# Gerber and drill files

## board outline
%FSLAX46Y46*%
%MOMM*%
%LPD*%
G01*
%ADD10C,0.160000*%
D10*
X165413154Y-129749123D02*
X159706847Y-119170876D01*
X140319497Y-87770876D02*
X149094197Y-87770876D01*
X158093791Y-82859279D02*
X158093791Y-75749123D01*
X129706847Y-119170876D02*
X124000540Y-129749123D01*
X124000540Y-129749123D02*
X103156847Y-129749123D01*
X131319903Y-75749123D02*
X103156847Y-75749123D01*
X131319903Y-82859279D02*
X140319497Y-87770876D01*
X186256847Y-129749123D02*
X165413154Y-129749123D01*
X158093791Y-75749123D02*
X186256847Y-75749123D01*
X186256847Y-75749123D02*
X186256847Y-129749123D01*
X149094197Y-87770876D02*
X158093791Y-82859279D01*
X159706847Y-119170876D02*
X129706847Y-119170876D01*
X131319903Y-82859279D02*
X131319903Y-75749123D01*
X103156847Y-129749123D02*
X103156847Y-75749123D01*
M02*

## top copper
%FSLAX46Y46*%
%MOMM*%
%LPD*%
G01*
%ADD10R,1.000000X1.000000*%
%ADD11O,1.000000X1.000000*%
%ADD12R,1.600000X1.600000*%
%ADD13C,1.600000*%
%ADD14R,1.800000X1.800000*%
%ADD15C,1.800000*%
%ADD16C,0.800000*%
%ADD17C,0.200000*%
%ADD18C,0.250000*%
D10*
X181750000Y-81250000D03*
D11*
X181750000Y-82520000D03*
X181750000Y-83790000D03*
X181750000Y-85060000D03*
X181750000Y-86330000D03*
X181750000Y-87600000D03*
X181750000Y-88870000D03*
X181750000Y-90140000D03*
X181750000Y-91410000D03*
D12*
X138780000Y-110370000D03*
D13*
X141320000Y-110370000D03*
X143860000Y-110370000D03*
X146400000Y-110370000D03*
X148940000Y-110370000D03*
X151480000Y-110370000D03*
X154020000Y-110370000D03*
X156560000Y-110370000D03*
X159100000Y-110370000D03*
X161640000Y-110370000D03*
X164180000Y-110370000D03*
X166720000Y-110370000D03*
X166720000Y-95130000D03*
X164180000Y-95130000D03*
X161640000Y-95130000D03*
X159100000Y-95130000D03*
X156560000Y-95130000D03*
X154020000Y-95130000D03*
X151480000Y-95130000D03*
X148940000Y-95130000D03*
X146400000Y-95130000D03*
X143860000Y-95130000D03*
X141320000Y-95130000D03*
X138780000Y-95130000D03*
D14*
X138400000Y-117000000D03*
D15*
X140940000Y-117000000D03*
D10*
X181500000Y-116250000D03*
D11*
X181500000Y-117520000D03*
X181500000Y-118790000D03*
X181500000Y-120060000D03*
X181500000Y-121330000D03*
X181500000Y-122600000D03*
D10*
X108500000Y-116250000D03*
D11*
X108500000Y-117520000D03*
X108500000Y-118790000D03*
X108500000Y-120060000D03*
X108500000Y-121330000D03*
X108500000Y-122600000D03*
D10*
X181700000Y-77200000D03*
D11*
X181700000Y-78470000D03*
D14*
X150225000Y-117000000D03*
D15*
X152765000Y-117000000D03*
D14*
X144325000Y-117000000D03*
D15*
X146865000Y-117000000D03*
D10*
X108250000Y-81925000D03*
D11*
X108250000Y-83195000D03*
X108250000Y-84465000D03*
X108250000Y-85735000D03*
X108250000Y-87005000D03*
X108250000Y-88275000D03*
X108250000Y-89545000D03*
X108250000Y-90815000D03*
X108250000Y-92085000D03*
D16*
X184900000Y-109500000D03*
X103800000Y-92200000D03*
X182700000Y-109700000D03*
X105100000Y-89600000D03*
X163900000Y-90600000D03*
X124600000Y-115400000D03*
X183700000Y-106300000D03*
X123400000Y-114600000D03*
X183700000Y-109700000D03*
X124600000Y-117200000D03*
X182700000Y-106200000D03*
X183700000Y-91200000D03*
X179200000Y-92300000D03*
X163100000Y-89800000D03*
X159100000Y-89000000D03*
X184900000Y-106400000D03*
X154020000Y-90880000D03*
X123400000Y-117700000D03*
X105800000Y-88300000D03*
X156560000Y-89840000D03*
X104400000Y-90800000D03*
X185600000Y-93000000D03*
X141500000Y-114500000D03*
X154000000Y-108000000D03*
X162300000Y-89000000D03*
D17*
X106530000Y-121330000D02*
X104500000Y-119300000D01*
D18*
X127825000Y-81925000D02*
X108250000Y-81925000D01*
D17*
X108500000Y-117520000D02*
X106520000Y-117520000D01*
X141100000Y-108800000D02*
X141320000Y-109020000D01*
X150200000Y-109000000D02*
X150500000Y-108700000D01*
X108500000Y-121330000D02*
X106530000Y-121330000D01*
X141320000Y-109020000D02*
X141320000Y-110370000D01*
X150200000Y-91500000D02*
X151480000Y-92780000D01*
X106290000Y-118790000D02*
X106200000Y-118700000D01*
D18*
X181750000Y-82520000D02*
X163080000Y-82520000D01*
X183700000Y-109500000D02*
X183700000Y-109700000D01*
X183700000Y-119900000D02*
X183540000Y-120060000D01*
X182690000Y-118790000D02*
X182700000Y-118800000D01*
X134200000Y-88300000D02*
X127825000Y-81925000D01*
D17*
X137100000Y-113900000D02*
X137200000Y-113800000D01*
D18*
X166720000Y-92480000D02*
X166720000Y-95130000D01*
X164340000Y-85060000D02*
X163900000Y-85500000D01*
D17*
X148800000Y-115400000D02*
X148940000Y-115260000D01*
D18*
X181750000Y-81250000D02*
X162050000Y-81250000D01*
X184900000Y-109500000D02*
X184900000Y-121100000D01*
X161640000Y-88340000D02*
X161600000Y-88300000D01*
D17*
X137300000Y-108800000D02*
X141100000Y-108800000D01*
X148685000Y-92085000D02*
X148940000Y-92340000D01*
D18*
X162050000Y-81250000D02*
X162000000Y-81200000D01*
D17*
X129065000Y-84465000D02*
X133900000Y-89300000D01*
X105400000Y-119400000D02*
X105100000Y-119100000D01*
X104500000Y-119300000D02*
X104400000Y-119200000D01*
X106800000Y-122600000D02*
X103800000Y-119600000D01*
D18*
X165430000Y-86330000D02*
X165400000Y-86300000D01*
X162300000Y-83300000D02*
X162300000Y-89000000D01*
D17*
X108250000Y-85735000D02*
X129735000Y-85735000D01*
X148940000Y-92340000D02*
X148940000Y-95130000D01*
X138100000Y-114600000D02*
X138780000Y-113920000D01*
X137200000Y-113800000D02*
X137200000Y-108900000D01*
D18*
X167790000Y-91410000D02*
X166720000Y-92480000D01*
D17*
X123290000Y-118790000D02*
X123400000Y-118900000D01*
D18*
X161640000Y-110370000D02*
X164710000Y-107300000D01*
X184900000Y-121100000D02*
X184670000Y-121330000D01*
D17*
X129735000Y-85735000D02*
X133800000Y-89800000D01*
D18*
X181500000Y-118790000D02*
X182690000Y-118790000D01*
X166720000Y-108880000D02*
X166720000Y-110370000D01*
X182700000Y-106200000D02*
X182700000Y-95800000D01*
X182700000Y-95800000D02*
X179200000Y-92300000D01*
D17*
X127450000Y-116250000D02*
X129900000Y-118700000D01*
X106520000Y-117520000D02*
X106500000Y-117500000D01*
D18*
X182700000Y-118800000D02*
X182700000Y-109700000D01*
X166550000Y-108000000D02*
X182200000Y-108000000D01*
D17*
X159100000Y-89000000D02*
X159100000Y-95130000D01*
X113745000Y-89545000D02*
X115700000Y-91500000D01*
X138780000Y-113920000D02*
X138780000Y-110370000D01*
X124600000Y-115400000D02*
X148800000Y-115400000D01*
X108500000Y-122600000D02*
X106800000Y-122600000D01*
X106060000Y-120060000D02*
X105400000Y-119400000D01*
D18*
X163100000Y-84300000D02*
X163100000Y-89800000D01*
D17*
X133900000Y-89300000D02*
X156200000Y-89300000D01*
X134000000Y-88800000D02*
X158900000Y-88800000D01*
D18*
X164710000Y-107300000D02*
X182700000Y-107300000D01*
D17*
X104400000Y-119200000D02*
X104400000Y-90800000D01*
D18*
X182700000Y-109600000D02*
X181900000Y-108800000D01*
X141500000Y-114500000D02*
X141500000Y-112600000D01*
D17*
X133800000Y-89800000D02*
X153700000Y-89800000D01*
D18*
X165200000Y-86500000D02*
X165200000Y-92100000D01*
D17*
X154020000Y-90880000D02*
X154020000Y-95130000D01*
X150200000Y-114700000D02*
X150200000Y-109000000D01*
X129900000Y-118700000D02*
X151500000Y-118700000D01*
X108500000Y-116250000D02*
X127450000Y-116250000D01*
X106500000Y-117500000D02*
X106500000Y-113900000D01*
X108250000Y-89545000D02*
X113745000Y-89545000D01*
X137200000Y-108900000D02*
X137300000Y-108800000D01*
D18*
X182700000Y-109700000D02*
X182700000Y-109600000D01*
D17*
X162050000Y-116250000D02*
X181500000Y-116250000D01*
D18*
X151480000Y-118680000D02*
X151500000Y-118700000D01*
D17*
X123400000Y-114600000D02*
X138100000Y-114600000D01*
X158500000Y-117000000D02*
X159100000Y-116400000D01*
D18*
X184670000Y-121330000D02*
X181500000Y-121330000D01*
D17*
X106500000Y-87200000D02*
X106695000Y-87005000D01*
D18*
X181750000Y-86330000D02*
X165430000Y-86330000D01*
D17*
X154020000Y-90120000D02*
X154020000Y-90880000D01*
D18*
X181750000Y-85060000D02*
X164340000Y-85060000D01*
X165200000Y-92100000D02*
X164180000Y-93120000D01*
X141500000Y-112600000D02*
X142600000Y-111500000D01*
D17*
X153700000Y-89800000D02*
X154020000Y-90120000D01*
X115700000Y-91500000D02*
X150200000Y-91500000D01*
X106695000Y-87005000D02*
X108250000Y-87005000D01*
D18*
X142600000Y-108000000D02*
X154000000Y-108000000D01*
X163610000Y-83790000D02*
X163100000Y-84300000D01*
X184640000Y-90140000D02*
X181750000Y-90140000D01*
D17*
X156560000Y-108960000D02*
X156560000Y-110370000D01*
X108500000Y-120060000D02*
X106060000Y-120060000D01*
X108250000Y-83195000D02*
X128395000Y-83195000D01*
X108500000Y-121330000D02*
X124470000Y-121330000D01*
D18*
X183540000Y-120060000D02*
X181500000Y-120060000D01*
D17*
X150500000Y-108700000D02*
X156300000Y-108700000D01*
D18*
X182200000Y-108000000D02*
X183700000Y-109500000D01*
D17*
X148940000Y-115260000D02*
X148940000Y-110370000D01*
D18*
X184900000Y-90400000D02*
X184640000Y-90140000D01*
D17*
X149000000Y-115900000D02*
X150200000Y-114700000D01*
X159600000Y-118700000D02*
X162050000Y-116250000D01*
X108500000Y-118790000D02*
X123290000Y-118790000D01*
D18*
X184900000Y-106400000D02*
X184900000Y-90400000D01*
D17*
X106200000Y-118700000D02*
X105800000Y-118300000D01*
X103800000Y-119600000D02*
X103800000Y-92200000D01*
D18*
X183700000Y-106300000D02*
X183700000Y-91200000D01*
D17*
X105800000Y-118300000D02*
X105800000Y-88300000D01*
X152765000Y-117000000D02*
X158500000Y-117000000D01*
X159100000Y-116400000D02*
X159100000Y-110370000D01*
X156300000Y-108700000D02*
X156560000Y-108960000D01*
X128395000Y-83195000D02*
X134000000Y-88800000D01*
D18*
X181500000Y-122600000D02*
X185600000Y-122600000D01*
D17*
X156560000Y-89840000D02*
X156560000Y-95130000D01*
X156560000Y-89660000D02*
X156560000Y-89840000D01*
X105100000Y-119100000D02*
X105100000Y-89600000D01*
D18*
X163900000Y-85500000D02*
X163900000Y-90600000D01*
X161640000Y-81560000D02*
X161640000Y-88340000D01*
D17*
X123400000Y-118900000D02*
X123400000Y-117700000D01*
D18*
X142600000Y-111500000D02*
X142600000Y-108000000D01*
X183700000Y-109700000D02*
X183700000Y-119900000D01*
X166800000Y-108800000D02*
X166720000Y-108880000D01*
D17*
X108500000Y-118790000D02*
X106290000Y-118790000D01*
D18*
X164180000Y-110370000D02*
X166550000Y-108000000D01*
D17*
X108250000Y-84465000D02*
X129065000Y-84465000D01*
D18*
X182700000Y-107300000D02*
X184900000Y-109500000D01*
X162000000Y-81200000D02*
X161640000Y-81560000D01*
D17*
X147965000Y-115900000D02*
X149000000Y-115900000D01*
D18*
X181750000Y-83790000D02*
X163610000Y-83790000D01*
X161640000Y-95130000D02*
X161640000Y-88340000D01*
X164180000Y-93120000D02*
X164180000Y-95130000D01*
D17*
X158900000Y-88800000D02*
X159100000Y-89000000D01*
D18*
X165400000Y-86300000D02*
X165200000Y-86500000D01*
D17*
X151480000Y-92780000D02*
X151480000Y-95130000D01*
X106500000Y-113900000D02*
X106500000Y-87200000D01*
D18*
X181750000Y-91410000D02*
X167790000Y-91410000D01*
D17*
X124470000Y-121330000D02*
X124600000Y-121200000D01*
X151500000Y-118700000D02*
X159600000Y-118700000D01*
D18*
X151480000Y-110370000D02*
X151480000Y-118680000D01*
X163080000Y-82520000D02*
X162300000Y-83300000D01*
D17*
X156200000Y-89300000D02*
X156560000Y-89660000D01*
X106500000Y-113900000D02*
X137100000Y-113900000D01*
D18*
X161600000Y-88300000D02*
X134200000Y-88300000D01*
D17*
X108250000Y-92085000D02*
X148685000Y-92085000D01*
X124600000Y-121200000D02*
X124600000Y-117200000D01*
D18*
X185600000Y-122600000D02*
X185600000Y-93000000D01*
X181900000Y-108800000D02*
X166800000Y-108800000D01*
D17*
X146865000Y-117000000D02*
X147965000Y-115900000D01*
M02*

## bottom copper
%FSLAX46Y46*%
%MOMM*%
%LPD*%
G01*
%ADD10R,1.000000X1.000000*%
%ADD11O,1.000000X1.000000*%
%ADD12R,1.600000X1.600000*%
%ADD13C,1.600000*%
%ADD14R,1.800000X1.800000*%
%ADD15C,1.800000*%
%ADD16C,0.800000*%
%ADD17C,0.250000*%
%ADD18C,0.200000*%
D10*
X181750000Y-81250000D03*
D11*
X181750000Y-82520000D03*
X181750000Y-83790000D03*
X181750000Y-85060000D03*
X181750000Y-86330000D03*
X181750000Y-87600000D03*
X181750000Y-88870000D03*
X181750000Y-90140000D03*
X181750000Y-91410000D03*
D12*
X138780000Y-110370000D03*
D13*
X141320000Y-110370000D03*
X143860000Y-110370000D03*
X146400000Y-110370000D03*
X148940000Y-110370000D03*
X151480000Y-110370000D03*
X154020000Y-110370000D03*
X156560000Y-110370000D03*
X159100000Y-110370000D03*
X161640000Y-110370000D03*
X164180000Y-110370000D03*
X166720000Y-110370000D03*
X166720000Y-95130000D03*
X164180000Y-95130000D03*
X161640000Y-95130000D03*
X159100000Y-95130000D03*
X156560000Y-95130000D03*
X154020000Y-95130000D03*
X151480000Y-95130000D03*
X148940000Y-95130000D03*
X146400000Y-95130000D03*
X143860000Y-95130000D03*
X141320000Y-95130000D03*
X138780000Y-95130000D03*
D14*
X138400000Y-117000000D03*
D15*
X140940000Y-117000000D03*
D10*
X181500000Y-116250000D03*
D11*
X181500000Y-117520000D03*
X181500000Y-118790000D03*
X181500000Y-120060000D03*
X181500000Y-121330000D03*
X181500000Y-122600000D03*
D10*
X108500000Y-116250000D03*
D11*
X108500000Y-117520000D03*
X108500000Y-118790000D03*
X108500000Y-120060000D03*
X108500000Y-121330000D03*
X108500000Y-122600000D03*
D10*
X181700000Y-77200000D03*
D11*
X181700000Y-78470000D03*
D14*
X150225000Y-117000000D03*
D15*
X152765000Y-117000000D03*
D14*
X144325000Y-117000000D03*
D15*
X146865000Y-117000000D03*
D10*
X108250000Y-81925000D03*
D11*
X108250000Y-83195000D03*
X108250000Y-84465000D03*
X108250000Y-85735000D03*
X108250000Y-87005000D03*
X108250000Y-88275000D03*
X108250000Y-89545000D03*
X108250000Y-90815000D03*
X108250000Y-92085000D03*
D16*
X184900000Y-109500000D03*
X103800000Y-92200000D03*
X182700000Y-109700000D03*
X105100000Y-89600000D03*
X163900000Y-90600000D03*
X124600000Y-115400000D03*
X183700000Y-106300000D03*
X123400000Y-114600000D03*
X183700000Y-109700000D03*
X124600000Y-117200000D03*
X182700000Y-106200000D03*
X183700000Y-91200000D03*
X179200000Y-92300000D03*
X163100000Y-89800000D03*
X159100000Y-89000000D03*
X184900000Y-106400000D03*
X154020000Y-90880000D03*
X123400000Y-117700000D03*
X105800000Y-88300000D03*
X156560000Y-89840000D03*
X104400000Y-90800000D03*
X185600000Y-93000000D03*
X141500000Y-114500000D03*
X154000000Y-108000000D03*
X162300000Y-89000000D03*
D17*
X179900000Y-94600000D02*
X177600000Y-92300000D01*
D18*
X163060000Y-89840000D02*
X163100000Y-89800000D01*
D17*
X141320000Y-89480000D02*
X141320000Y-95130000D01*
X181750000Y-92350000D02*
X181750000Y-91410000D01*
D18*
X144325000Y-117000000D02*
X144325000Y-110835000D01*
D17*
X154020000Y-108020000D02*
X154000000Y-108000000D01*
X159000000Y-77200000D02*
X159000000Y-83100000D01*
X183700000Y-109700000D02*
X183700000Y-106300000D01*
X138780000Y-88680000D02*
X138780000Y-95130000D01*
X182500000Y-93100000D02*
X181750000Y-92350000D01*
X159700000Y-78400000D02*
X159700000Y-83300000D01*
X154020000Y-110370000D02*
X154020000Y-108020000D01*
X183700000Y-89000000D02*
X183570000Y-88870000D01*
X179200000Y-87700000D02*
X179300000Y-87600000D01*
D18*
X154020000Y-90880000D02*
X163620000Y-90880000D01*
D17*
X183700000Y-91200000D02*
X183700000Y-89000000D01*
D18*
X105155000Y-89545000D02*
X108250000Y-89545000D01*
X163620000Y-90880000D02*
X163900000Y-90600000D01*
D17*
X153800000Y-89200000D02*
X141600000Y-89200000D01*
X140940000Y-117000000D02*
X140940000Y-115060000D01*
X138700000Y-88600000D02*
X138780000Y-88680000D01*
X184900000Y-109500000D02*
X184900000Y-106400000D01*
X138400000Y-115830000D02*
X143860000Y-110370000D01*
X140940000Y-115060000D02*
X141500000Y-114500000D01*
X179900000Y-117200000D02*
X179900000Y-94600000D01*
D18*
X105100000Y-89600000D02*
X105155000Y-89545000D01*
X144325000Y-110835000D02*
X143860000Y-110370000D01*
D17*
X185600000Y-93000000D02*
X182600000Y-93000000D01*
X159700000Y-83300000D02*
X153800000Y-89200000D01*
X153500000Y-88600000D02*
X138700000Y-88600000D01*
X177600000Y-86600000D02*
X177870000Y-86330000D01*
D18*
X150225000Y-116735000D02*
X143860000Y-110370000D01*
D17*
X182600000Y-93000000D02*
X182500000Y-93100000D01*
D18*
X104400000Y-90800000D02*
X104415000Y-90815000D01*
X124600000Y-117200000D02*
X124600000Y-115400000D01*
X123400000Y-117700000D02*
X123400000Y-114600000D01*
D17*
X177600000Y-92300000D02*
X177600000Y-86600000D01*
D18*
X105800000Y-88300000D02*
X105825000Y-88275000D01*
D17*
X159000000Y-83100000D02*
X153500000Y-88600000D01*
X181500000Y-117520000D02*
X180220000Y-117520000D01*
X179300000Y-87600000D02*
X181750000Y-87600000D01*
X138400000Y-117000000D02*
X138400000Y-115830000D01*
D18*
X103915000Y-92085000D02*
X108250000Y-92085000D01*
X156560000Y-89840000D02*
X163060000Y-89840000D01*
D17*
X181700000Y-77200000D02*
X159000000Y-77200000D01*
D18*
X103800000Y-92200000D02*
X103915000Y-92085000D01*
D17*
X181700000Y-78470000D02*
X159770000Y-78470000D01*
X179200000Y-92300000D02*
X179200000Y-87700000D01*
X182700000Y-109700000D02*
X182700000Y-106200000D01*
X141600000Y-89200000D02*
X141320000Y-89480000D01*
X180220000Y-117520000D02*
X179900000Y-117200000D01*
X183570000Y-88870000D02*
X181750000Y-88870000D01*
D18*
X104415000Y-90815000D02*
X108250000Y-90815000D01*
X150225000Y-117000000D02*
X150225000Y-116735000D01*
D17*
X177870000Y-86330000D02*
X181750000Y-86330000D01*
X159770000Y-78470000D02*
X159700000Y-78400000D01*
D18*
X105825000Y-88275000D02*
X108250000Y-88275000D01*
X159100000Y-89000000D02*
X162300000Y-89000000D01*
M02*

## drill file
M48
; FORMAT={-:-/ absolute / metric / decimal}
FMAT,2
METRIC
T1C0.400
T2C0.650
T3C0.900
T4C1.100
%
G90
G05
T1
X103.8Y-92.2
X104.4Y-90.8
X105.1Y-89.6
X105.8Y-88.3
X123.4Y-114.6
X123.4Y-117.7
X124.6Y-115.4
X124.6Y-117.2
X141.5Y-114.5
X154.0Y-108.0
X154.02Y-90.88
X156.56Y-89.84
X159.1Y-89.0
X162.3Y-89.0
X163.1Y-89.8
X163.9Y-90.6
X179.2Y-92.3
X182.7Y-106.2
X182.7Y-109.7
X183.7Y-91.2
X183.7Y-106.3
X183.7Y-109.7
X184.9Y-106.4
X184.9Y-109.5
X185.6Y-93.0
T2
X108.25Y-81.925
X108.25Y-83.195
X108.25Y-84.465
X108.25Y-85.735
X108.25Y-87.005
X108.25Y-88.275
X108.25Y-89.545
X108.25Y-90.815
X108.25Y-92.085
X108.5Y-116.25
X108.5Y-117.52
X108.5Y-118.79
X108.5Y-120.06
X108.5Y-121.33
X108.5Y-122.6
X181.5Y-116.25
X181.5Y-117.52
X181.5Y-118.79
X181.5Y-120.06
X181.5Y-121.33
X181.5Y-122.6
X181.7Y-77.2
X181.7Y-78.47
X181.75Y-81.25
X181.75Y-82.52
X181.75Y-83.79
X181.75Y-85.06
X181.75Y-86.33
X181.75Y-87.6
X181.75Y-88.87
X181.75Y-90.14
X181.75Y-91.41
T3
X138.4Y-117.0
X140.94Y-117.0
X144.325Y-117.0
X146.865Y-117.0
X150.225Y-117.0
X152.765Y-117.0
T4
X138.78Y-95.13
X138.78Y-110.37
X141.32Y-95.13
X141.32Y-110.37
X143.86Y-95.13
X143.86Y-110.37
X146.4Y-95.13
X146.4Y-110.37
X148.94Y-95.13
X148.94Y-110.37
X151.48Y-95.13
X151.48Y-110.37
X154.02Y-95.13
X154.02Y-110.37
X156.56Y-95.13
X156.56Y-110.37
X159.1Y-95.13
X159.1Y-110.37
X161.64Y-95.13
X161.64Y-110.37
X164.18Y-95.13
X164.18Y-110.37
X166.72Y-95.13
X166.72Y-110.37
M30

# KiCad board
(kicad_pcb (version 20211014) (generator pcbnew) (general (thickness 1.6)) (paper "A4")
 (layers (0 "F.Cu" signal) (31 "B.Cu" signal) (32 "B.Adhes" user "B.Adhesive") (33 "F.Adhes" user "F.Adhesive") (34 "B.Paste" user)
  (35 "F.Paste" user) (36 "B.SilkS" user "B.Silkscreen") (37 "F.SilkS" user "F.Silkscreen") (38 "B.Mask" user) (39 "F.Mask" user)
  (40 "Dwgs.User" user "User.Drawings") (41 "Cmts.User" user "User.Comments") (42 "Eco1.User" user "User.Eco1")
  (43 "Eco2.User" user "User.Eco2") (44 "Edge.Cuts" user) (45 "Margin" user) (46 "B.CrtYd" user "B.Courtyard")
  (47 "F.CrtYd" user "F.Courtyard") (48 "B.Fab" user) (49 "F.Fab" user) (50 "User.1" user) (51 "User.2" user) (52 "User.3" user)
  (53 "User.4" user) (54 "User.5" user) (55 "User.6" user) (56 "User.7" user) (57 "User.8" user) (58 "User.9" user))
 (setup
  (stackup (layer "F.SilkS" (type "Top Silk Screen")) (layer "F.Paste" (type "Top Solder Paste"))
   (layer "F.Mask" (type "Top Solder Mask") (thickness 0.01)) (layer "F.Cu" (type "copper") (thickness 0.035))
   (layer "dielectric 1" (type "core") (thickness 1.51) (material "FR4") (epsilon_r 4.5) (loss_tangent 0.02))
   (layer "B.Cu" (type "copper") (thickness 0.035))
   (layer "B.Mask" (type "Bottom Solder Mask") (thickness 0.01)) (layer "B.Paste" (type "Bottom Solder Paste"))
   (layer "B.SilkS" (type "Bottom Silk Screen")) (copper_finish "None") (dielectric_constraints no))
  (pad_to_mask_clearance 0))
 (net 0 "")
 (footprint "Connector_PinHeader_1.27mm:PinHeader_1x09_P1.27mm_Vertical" (layer "F.Cu") (at 181.75 81.25)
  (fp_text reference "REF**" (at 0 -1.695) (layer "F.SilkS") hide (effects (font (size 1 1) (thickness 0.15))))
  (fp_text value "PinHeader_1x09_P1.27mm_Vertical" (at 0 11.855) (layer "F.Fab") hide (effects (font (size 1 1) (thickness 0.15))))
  (pad "1" thru_hole rect (at 0 0) (size 1 1) (drill 0.65) (layers *.Cu *.Mask))
  (pad "2" thru_hole oval (at 0 1.27) (size 1 1) (drill 0.65) (layers *.Cu *.Mask))
  (pad "3" thru_hole oval (at 0 2.54) (size 1 1) (drill 0.65) (layers *.Cu *.Mask))
  (pad "4" thru_hole oval (at 0 3.81) (size 1 1) (drill 0.65) (layers *.Cu *.Mask))
  (pad "5" thru_hole oval (at 0 5.08) (size 1 1) (drill 0.65) (layers *.Cu *.Mask))
  (pad "6" thru_hole oval (at 0 6.35) (size 1 1) (drill 0.65) (layers *.Cu *.Mask))
  (pad "7" thru_hole oval (at 0 7.62) (size 1 1) (drill 0.65) (layers *.Cu *.Mask))
  (pad "8" thru_hole oval (at 0 8.89) (size 1 1) (drill 0.65) (layers *.Cu *.Mask))
  (pad "9" thru_hole oval (at 0 10.16) (size 1 1) (drill 0.65) (layers *.Cu *.Mask)))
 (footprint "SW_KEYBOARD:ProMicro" (layer "F.Cu") (at 152.75 102.75)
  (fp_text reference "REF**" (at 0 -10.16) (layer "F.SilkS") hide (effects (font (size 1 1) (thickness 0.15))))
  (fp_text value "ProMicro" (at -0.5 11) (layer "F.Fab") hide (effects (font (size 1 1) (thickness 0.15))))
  (pad "1" thru_hole rect locked (at -13.97 7.62) (size 1.6 1.6) (drill 1.1) (layers *.Cu *.Mask "F.SilkS"))
  (pad "2" thru_hole circle locked (at -11.43 7.62) (size 1.6 1.6) (drill 1.1) (layers *.Cu *.Mask "F.SilkS"))
  (pad "3" thru_hole circle locked (at -8.89 7.62) (size 1.6 1.6) (drill 1.1) (layers *.Cu *.Mask "F.SilkS"))
  (pad "4" thru_hole circle locked (at -6.35 7.62) (size 1.6 1.6) (drill 1.1) (layers *.Cu *.Mask "F.SilkS"))
  (pad "5" thru_hole circle locked (at -3.81 7.62) (size 1.6 1.6) (drill 1.1) (layers *.Cu *.Mask "F.SilkS"))
  (pad "6" thru_hole circle locked (at -1.27 7.62) (size 1.6 1.6) (drill 1.1) (layers *.Cu *.Mask "F.SilkS"))
  (pad "7" thru_hole circle locked (at 1.27 7.62) (size 1.6 1.6) (drill 1.1) (layers *.Cu *.Mask "F.SilkS"))
  (pad "8" thru_hole circle locked (at 3.81 7.62) (size 1.6 1.6) (drill 1.1) (layers *.Cu *.Mask "F.SilkS"))
  (pad "9" thru_hole circle locked (at 6.35 7.62) (size 1.6 1.6) (drill 1.1) (layers *.Cu *.Mask "F.SilkS"))
  (pad "10" thru_hole circle locked (at 8.89 7.62) (size 1.6 1.6) (drill 1.1) (layers *.Cu *.Mask "F.SilkS"))
  (pad "11" thru_hole circle locked (at 11.43 7.62) (size 1.6 1.6) (drill 1.1) (layers *.Cu *.Mask "F.SilkS"))
  (pad "12" thru_hole circle locked (at 13.97 7.62) (size 1.6 1.6) (drill 1.1) (layers *.Cu *.Mask "F.SilkS"))
  (pad "13" thru_hole circle locked (at 13.97 -7.62) (size 1.6 1.6) (drill 1.1) (layers *.Cu *.Mask "F.SilkS"))
  (pad "14" thru_hole circle locked (at 11.43 -7.62) (size 1.6 1.6) (drill 1.1) (layers *.Cu *.Mask "F.SilkS"))
  (pad "15" thru_hole circle locked (at 8.89 -7.62) (size 1.6 1.6) (drill 1.1) (layers *.Cu *.Mask "F.SilkS"))
  (pad "16" thru_hole circle locked (at 6.35 -7.62) (size 1.6 1.6) (drill 1.1) (layers *.Cu *.Mask "F.SilkS"))
  (pad "17" thru_hole circle locked (at 3.81 -7.62) (size 1.6 1.6) (drill 1.1) (layers *.Cu *.Mask "F.SilkS"))
  (pad "18" thru_hole circle locked (at 1.27 -7.62) (size 1.6 1.6) (drill 1.1) (layers *.Cu *.Mask "F.SilkS"))
  (pad "19" thru_hole circle locked (at -1.27 -7.62) (size 1.6 1.6) (drill 1.1) (layers *.Cu *.Mask "F.SilkS"))
  (pad "20" thru_hole circle locked (at -3.81 -7.62) (size 1.6 1.6) (drill 1.1) (layers *.Cu *.Mask "F.SilkS"))
  (pad "21" thru_hole circle locked (at -6.35 -7.62) (size 1.6 1.6) (drill 1.1) (layers *.Cu *.Mask "F.SilkS"))
  (pad "22" thru_hole circle locked (at -8.89 -7.62) (size 1.6 1.6) (drill 1.1) (layers *.Cu *.Mask "F.SilkS"))
  (pad "23" thru_hole circle locked (at -11.43 -7.62) (size 1.6 1.6) (drill 1.1) (layers *.Cu *.Mask "F.SilkS"))
  (pad "24" thru_hole circle locked (at -13.97 -7.62) (size 1.6 1.6) (drill 1.1) (layers *.Cu *.Mask "F.SilkS")))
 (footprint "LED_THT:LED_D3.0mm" (layer "F.Cu") (at 138.4 117)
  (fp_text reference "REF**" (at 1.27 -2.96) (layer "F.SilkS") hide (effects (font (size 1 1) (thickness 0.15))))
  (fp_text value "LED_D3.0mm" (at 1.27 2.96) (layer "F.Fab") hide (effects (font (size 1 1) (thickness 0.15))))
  (pad "1" thru_hole rect (at 0 0) (size 1.8 1.8) (drill 0.9) (layers *.Cu *.Mask))
  (pad "2" thru_hole circle (at 2.54 0) (size 1.8 1.8) (drill 0.9) (layers *.Cu *.Mask)))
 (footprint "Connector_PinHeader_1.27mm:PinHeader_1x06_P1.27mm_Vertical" (layer "F.Cu") (at 181.5 116.25)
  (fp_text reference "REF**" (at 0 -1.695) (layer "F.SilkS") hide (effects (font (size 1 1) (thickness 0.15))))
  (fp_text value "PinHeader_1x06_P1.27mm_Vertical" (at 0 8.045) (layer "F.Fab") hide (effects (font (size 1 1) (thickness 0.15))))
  (pad "1" thru_hole rect (at 0 0) (size 1 1) (drill 0.65) (layers *.Cu *.Mask))
  (pad "2" thru_hole oval (at 0 1.27) (size 1 1) (drill 0.65) (layers *.Cu *.Mask))
  (pad "3" thru_hole oval (at 0 2.54) (size 1 1) (drill 0.65) (layers *.Cu *.Mask))
  (pad "4" thru_hole oval (at 0 3.81) (size 1 1) (drill 0.65) (layers *.Cu *.Mask))
  (pad "5" thru_hole oval (at 0 5.08) (size 1 1) (drill 0.65) (layers *.Cu *.Mask))
  (pad "6" thru_hole oval (at 0 6.35) (size 1 1) (drill 0.65) (layers *.Cu *.Mask)))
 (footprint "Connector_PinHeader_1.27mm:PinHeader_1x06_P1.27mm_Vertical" (layer "F.Cu") (at 108.5 116.25)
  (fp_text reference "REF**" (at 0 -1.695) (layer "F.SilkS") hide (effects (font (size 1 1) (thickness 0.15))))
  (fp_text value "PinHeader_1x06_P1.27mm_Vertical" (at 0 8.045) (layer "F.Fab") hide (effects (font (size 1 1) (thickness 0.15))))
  (pad "1" thru_hole rect (at 0 0) (size 1 1) (drill 0.65) (layers *.Cu *.Mask))
  (pad "2" thru_hole oval (at 0 1.27) (size 1 1) (drill 0.65) (layers *.Cu *.Mask))
  (pad "3" thru_hole oval (at 0 2.54) (size 1 1) (drill 0.65) (layers *.Cu *.Mask))
  (pad "4" thru_hole oval (at 0 3.81) (size 1 1) (drill 0.65) (layers *.Cu *.Mask))
  (pad "5" thru_hole oval (at 0 5.08) (size 1 1) (drill 0.65) (layers *.Cu *.Mask))
  (pad "6" thru_hole oval (at 0 6.35) (size 1 1) (drill 0.65) (layers *.Cu *.Mask)))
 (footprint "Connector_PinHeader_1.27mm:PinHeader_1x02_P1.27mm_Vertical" (layer "F.Cu") (at 181.7 77.2)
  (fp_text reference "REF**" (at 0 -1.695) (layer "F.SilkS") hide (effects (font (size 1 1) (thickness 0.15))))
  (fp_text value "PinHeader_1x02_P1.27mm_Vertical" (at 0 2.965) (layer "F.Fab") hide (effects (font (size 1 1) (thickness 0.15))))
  (pad "1" thru_hole rect (at 0 0) (size 1 1) (drill 0.65) (layers *.Cu *.Mask))
  (pad "2" thru_hole oval (at 0 1.27) (size 1 1) (drill 0.65) (layers *.Cu *.Mask)))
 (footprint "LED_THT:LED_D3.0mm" (layer "F.Cu") (at 150.225 117)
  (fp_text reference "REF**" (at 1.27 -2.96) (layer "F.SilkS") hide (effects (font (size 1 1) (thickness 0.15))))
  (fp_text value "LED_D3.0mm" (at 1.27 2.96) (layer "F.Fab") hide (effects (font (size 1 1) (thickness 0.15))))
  (pad "1" thru_hole rect (at 0 0) (size 1.8 1.8) (drill 0.9) (layers *.Cu *.Mask))
  (pad "2" thru_hole circle (at 2.54 0) (size 1.8 1.8) (drill 0.9) (layers *.Cu *.Mask)))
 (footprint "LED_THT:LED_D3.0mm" (layer "F.Cu") (at 144.325 117)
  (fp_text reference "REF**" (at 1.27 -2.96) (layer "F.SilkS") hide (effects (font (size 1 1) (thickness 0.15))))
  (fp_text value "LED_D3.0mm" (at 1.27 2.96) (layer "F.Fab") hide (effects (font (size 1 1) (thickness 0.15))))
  (pad "1" thru_hole rect (at 0 0) (size 1.8 1.8) (drill 0.9) (layers *.Cu *.Mask))
  (pad "2" thru_hole circle (at 2.54 0) (size 1.8 1.8) (drill 0.9) (layers *.Cu *.Mask)))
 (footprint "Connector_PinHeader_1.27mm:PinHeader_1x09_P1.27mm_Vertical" (layer "F.Cu") (at 108.25 81.925)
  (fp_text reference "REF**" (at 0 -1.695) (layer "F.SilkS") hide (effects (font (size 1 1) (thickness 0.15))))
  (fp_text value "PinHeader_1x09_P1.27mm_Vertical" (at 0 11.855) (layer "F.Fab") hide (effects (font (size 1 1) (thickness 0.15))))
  (pad "1" thru_hole rect (at 0 0) (size 1 1) (drill 0.65) (layers *.Cu *.Mask))
  (pad "2" thru_hole oval (at 0 1.27) (size 1 1) (drill 0.65) (layers *.Cu *.Mask))
  (pad "3" thru_hole oval (at 0 2.54) (size 1 1) (drill 0.65) (layers *.Cu *.Mask))
  (pad "4" thru_hole oval (at 0 3.81) (size 1 1) (drill 0.65) (layers *.Cu *.Mask))
  (pad "5" thru_hole oval (at 0 5.08) (size 1 1) (drill 0.65) (layers *.Cu *.Mask))
  (pad "6" thru_hole oval (at 0 6.35) (size 1 1) (drill 0.65) (layers *.Cu *.Mask))
  (pad "7" thru_hole oval (at 0 7.62) (size 1 1) (drill 0.65) (layers *.Cu *.Mask))
  (pad "8" thru_hole oval (at 0 8.89) (size 1 1) (drill 0.65) (layers *.Cu *.Mask))
  (pad "9" thru_hole oval (at 0 10.16) (size 1 1) (drill 0.65) (layers *.Cu *.Mask)))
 (gr_line (start 165.413154 129.749123) (end 159.706847 119.170876) (layer "Edge.Cuts") (width 0.16))
 (gr_line (start 140.319497 87.770876) (end 149.094197 87.770876) (layer "Edge.Cuts") (width 0.16))
 (gr_line (start 158.093791 82.859279) (end 158.093791 75.749123) (layer "Edge.Cuts") (width 0.16))
 (gr_line (start 129.706847 119.170876) (end 124.00054 129.749123) (layer "Edge.Cuts") (width 0.16))
 (gr_line (start 124.00054 129.749123) (end 103.156847 129.749123) (layer "Edge.Cuts") (width 0.16))
 (gr_line (start 131.319903 75.749123) (end 103.156847 75.749123) (layer "Edge.Cuts") (width 0.16))
 (gr_line (start 131.319903 82.859279) (end 140.319497 87.770876) (layer "Edge.Cuts") (width 0.16))
 (gr_line (start 186.256847 129.749123) (end 165.413154 129.749123) (layer "Edge.Cuts") (width 0.16))
 (gr_line (start 158.093791 75.749123) (end 186.256847 75.749123) (layer "Edge.Cuts") (width 0.16))
 (gr_line (start 186.256847 75.749123) (end 186.256847 129.749123) (layer "Edge.Cuts") (width 0.16))
 (gr_line (start 149.094197 87.770876) (end 158.093791 82.859279) (layer "Edge.Cuts") (width 0.16))
 (gr_line (start 159.706847 119.170876) (end 129.706847 119.170876) (layer "Edge.Cuts") (width 0.16))
 (gr_line (start 131.319903 82.859279) (end 131.319903 75.749123) (layer "Edge.Cuts") (width 0.16))
 (gr_line (start 103.156847 129.749123) (end 103.156847 75.749123) (layer "Edge.Cuts") (width 0.16))
 (segment (start 106.53 121.33) (end 104.5 119.3) (width 0.2) (layer "F.Cu") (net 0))
 (segment (start 127.825 81.925) (end 108.25 81.925) (width 0.25) (layer "F.Cu") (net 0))
 (segment (start 108.5 117.52) (end 106.52 117.52) (width 0.2) (layer "F.Cu") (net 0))
 (segment (start 141.1 108.8) (end 141.32 109.02) (width 0.2) (layer "F.Cu") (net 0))
 (segment (start 150.2 109) (end 150.5 108.7) (width 0.2) (layer "F.Cu") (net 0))
 (segment (start 108.5 121.33) (end 106.53 121.33) (width 0.2) (layer "F.Cu") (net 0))
 (segment (start 141.32 109.02) (end 141.32 110.37) (width 0.2) (layer "F.Cu") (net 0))
 (segment (start 150.2 91.5) (end 151.48 92.78) (width 0.2) (layer "F.Cu") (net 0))
 (segment (start 106.29 118.79) (end 106.2 118.7) (width 0.2) (layer "F.Cu") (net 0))
 (segment (start 181.75 82.52) (end 163.08 82.52) (width 0.25) (layer "F.Cu") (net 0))
 (segment (start 183.7 109.5) (end 183.7 109.7) (width 0.25) (layer "F.Cu") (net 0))
 (segment (start 183.7 119.9) (end 183.54 120.06) (width 0.25) (layer "F.Cu") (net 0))
 (segment (start 182.69 118.79) (end 182.7 118.8) (width 0.25) (layer "F.Cu") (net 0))
 (segment (start 134.2 88.3) (end 127.825 81.925) (width 0.25) (layer "F.Cu") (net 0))
 (segment (start 137.1 113.9) (end 137.2 113.8) (width 0.2) (layer "F.Cu") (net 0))
 (segment (start 166.72 92.48) (end 166.72 95.13) (width 0.25) (layer "F.Cu") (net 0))
 (segment (start 164.34 85.06) (end 163.9 85.5) (width 0.25) (layer "F.Cu") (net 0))
 (segment (start 148.8 115.4) (end 148.94 115.26) (width 0.2) (layer "F.Cu") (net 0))
 (segment (start 181.75 81.25) (end 162.05 81.25) (width 0.25) (layer "F.Cu") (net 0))
 (segment (start 184.9 109.5) (end 184.9 121.1) (width 0.25) (layer "F.Cu") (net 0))
 (segment (start 161.64 88.34) (end 161.6 88.3) (width 0.25) (layer "F.Cu") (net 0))
 (segment (start 137.3 108.8) (end 141.1 108.8) (width 0.2) (layer "F.Cu") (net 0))
 (segment (start 148.685 92.085) (end 148.94 92.34) (width 0.2) (layer "F.Cu") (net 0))
 (segment (start 162.05 81.25) (end 162 81.2) (width 0.25) (layer "F.Cu") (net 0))
 (segment (start 129.065 84.465) (end 133.9 89.3) (width 0.2) (layer "F.Cu") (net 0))
 (segment (start 105.4 119.4) (end 105.1 119.1) (width 0.2) (layer "F.Cu") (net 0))
 (segment (start 104.5 119.3) (end 104.4 119.2) (width 0.2) (layer "F.Cu") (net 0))
 (segment (start 106.8 122.6) (end 103.8 119.6) (width 0.2) (layer "F.Cu") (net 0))
 (segment (start 165.43 86.33) (end 165.4 86.3) (width 0.25) (layer "F.Cu") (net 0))
 (segment (start 162.3 83.3) (end 162.3 89) (width 0.25) (layer "F.Cu") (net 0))
 (segment (start 108.25 85.735) (end 129.735 85.735) (width 0.2) (layer "F.Cu") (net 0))
 (segment (start 148.94 92.34) (end 148.94 95.13) (width 0.2) (layer "F.Cu") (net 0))
 (segment (start 138.1 114.6) (end 138.78 113.92) (width 0.2) (layer "F.Cu") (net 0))
 (segment (start 137.2 113.8) (end 137.2 108.9) (width 0.2) (layer "F.Cu") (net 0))
 (segment (start 167.79 91.41) (end 166.72 92.48) (width 0.25) (layer "F.Cu") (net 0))
 (segment (start 123.29 118.79) (end 123.4 118.9) (width 0.2) (layer "F.Cu") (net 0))
 (segment (start 161.64 110.37) (end 164.71 107.3) (width 0.25) (layer "F.Cu") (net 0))
 (segment (start 184.9 121.1) (end 184.67 121.33) (width 0.25) (layer "F.Cu") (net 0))
 (segment (start 129.735 85.735) (end 133.8 89.8) (width 0.2) (layer "F.Cu") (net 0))
 (segment (start 181.5 118.79) (end 182.69 118.79) (width 0.25) (layer "F.Cu") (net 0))
 (segment (start 166.72 108.88) (end 166.72 110.37) (width 0.25) (layer "F.Cu") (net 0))
 (segment (start 182.7 106.2) (end 182.7 95.8) (width 0.25) (layer "F.Cu") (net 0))
 (segment (start 182.7 95.8) (end 179.2 92.3) (width 0.25) (layer "F.Cu") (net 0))
 (segment (start 127.45 116.25) (end 129.9 118.7) (width 0.2) (layer "F.Cu") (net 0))
 (segment (start 106.52 117.52) (end 106.5 117.5) (width 0.2) (layer "F.Cu") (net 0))
 (segment (start 182.7 118.8) (end 182.7 109.7) (width 0.25) (layer "F.Cu") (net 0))
 (segment (start 166.55 108) (end 182.2 108) (width 0.25) (layer "F.Cu") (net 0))
 (segment (start 159.1 89) (end 159.1 95.13) (width 0.2) (layer "F.Cu") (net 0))
 (segment (start 113.745 89.545) (end 115.7 91.5) (width 0.2) (layer "F.Cu") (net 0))
 (segment (start 138.78 113.92) (end 138.78 110.37) (width 0.2) (layer "F.Cu") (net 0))
 (segment (start 124.6 115.4) (end 148.8 115.4) (width 0.2) (layer "F.Cu") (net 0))
 (segment (start 108.5 122.6) (end 106.8 122.6) (width 0.2) (layer "F.Cu") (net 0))
 (segment (start 106.06 120.06) (end 105.4 119.4) (width 0.2) (layer "F.Cu") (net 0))
 (segment (start 163.1 84.3) (end 163.1 89.8) (width 0.25) (layer "F.Cu") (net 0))
 (segment (start 133.9 89.3) (end 156.2 89.3) (width 0.2) (layer "F.Cu") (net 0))
 (segment (start 134 88.8) (end 158.9 88.8) (width 0.2) (layer "F.Cu") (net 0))
 (segment (start 164.71 107.3) (end 182.7 107.3) (width 0.25) (layer "F.Cu") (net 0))
 (segment (start 104.4 119.2) (end 104.4 90.8) (width 0.2) (layer "F.Cu") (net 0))
 (segment (start 182.7 109.6) (end 181.9 108.8) (width 0.25) (layer "F.Cu") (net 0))
 (segment (start 141.5 114.5) (end 141.5 112.6) (width 0.25) (layer "F.Cu") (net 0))
 (segment (start 133.8 89.8) (end 153.7 89.8) (width 0.2) (layer "F.Cu") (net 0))
 (segment (start 165.2 86.5) (end 165.2 92.1) (width 0.25) (layer "F.Cu") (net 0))
 (segment (start 154.02 90.88) (end 154.02 95.13) (width 0.2) (layer "F.Cu") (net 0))
 (segment (start 150.2 114.7) (end 150.2 109) (width 0.2) (layer "F.Cu") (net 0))
 (segment (start 129.9 118.7) (end 151.5 118.7) (width 0.2) (layer "F.Cu") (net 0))
 (segment (start 108.5 116.25) (end 127.45 116.25) (width 0.2) (layer "F.Cu") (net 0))
 (segment (start 106.5 117.5) (end 106.5 113.9) (width 0.2) (layer "F.Cu") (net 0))
 (segment (start 108.25 89.545) (end 113.745 89.545) (width 0.2) (layer "F.Cu") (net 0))
 (segment (start 137.2 108.9) (end 137.3 108.8) (width 0.2) (layer "F.Cu") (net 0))
 (segment (start 182.7 109.7) (end 182.7 109.6) (width 0.25) (layer "F.Cu") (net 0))
 (segment (start 162.05 116.25) (end 181.5 116.25) (width 0.2) (layer "F.Cu") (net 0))
 (segment (start 151.48 118.68) (end 151.5 118.7) (width 0.25) (layer "F.Cu") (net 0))
 (segment (start 123.4 114.6) (end 138.1 114.6) (width 0.2) (layer "F.Cu") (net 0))
 (segment (start 158.5 117) (end 159.1 116.4) (width 0.2) (layer "F.Cu") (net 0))
 (segment (start 184.67 121.33) (end 181.5 121.33) (width 0.25) (layer "F.Cu") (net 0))
 (segment (start 106.5 87.2) (end 106.695 87.005) (width 0.2) (layer "F.Cu") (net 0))
 (segment (start 181.75 86.33) (end 165.43 86.33) (width 0.25) (layer "F.Cu") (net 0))
 (segment (start 154.02 90.12) (end 154.02 90.88) (width 0.2) (layer "F.Cu") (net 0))
 (segment (start 181.75 85.06) (end 164.34 85.06) (width 0.25) (layer "F.Cu") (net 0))
 (segment (start 165.2 92.1) (end 164.18 93.12) (width 0.25) (layer "F.Cu") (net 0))
 (segment (start 141.5 112.6) (end 142.6 111.5) (width 0.25) (layer "F.Cu") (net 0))
 (segment (start 153.7 89.8) (end 154.02 90.12) (width 0.2) (layer "F.Cu") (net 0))
 (segment (start 115.7 91.5) (end 150.2 91.5) (width 0.2) (layer "F.Cu") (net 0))
 (segment (start 106.695 87.005) (end 108.25 87.005) (width 0.2) (layer "F.Cu") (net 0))
 (segment (start 142.6 108) (end 154 108) (width 0.25) (layer "F.Cu") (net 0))
 (segment (start 163.61 83.79) (end 163.1 84.3) (width 0.25) (layer "F.Cu") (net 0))
 (segment (start 184.64 90.14) (end 181.75 90.14) (width 0.25) (layer "F.Cu") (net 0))
 (segment (start 156.56 108.96) (end 156.56 110.37) (width 0.2) (layer "F.Cu") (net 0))
 (segment (start 108.5 120.06) (end 106.06 120.06) (width 0.2) (layer "F.Cu") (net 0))
 (segment (start 108.25 83.195) (end 128.395 83.195) (width 0.2) (layer "F.Cu") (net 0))
 (segment (start 108.5 121.33) (end 124.47 121.33) (width 0.2) (layer "F.Cu") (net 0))
 (segment (start 183.54 120.06) (end 181.5 120.06) (width 0.25) (layer "F.Cu") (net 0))
 (segment (start 150.5 108.7) (end 156.3 108.7) (width 0.2) (layer "F.Cu") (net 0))
 (segment (start 182.2 108) (end 183.7 109.5) (width 0.25) (layer "F.Cu") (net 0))
 (segment (start 148.94 115.26) (end 148.94 110.37) (width 0.2) (layer "F.Cu") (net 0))
 (segment (start 184.9 90.4) (end 184.64 90.14) (width 0.25) (layer "F.Cu") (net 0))
 (segment (start 149 115.9) (end 150.2 114.7) (width 0.2) (layer "F.Cu") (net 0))
 (segment (start 159.6 118.7) (end 162.05 116.25) (width 0.2) (layer "F.Cu") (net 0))
 (segment (start 108.5 118.79) (end 123.29 118.79) (width 0.2) (layer "F.Cu") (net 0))
 (segment (start 184.9 106.4) (end 184.9 90.4) (width 0.25) (layer "F.Cu") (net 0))
 (segment (start 106.2 118.7) (end 105.8 118.3) (width 0.2) (layer "F.Cu") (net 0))
 (segment (start 103.8 119.6) (end 103.8 92.2) (width 0.2) (layer "F.Cu") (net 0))
 (segment (start 183.7 106.3) (end 183.7 91.2) (width 0.25) (layer "F.Cu") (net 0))
 (segment (start 105.8 118.3) (end 105.8 88.3) (width 0.2) (layer "F.Cu") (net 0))
 (segment (start 152.765 117) (end 158.5 117) (width 0.2) (layer "F.Cu") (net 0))
 (segment (start 159.1 116.4) (end 159.1 110.37) (width 0.2) (layer "F.Cu") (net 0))
 (segment (start 156.3 108.7) (end 156.56 108.96) (width 0.2) (layer "F.Cu") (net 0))
 (segment (start 128.395 83.195) (end 134 88.8) (width 0.2) (layer "F.Cu") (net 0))
 (segment (start 181.5 122.6) (end 185.6 122.6) (width 0.25) (layer "F.Cu") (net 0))
 (segment (start 156.56 89.84) (end 156.56 95.13) (width 0.2) (layer "F.Cu") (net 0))
 (segment (start 156.56 89.66) (end 156.56 89.84) (width 0.2) (layer "F.Cu") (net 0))
 (segment (start 105.1 119.1) (end 105.1 89.6) (width 0.2) (layer "F.Cu") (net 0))
 (segment (start 163.9 85.5) (end 163.9 90.6) (width 0.25) (layer "F.Cu") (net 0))
 (segment (start 161.64 81.56) (end 161.64 88.34) (width 0.25) (layer "F.Cu") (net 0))
 (segment (start 123.4 118.9) (end 123.4 117.7) (width 0.2) (layer "F.Cu") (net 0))
 (segment (start 142.6 111.5) (end 142.6 108) (width 0.25) (layer "F.Cu") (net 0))
 (segment (start 183.7 109.7) (end 183.7 119.9) (width 0.25) (layer "F.Cu") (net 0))
 (segment (start 166.8 108.8) (end 166.72 108.88) (width 0.25) (layer "F.Cu") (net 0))
 (segment (start 108.5 118.79) (end 106.29 118.79) (width 0.2) (layer "F.Cu") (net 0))
 (segment (start 164.18 110.37) (end 166.55 108) (width 0.25) (layer "F.Cu") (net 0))
 (segment (start 108.25 84.465) (end 129.065 84.465) (width 0.2) (layer "F.Cu") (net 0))
 (segment (start 182.7 107.3) (end 184.9 109.5) (width 0.25) (layer "F.Cu") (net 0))
 (segment (start 162 81.2) (end 161.64 81.56) (width 0.25) (layer "F.Cu") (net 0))
 (segment (start 147.965 115.9) (end 149 115.9) (width 0.2) (layer "F.Cu") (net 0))
 (segment (start 181.75 83.79) (end 163.61 83.79) (width 0.25) (layer "F.Cu") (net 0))
 (segment (start 161.64 95.13) (end 161.64 88.34) (width 0.25) (layer "F.Cu") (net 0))
 (segment (start 164.18 93.12) (end 164.18 95.13) (width 0.25) (layer "F.Cu") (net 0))
 (segment (start 158.9 88.8) (end 159.1 89) (width 0.2) (layer "F.Cu") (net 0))
 (segment (start 165.4 86.3) (end 165.2 86.5) (width 0.25) (layer "F.Cu") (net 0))
 (segment (start 151.48 92.78) (end 151.48 95.13) (width 0.2) (layer "F.Cu") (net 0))
 (segment (start 106.5 113.9) (end 106.5 87.2) (width 0.2) (layer "F.Cu") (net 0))
 (segment (start 181.75 91.41) (end 167.79 91.41) (width 0.25) (layer "F.Cu") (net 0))
 (segment (start 124.47 121.33) (end 124.6 121.2) (width 0.2) (layer "F.Cu") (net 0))
 (segment (start 151.5 118.7) (end 159.6 118.7) (width 0.2) (layer "F.Cu") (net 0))
 (segment (start 151.48 110.37) (end 151.48 118.68) (width 0.25) (layer "F.Cu") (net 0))
 (segment (start 163.08 82.52) (end 162.3 83.3) (width 0.25) (layer "F.Cu") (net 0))
 (segment (start 156.2 89.3) (end 156.56 89.66) (width 0.2) (layer "F.Cu") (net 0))
 (segment (start 106.5 113.9) (end 137.1 113.9) (width 0.2) (layer "F.Cu") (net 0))
 (segment (start 161.6 88.3) (end 134.2 88.3) (width 0.25) (layer "F.Cu") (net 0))
 (segment (start 108.25 92.085) (end 148.685 92.085) (width 0.2) (layer "F.Cu") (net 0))
 (segment (start 124.6 121.2) (end 124.6 117.2) (width 0.2) (layer "F.Cu") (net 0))
 (segment (start 185.6 122.6) (end 185.6 93) (width 0.25) (layer "F.Cu") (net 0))
 (segment (start 181.9 108.8) (end 166.8 108.8) (width 0.25) (layer "F.Cu") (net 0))
 (segment (start 146.865 117) (end 147.965 115.9) (width 0.2) (layer "F.Cu") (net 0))
 (via (at 184.9 109.5) (size 0.8) (drill 0.4) (layers "F.Cu" "B.Cu") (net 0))
 (via (at 103.8 92.2) (size 0.8) (drill 0.4) (layers "F.Cu" "B.Cu") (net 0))
 (via (at 182.7 109.7) (size 0.8) (drill 0.4) (layers "F.Cu" "B.Cu") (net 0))
 (via (at 105.1 89.6) (size 0.8) (drill 0.4) (layers "F.Cu" "B.Cu") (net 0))
 (via (at 163.9 90.6) (size 0.8) (drill 0.4) (layers "F.Cu" "B.Cu") (free) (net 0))
 (via (at 124.6 115.4) (size 0.8) (drill 0.4) (layers "F.Cu" "B.Cu") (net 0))
 (via (at 183.7 106.3) (size 0.8) (drill 0.4) (layers "F.Cu" "B.Cu") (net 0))
 (via (at 123.4 114.6) (size 0.8) (drill 0.4) (layers "F.Cu" "B.Cu") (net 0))
 (via (at 183.7 109.7) (size 0.8) (drill 0.4) (layers "F.Cu" "B.Cu") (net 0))
 (via (at 124.6 117.2) (size 0.8) (drill 0.4) (layers "F.Cu" "B.Cu") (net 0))
 (via (at 182.7 106.2) (size 0.8) (drill 0.4) (layers "F.Cu" "B.Cu") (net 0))
 (via (at 183.7 91.2) (size 0.8) (drill 0.4) (layers "F.Cu" "B.Cu") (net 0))
 (via (at 179.2 92.3) (size 0.8) (drill 0.4) (layers "F.Cu" "B.Cu") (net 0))
 (via (at 163.1 89.8) (size 0.8) (drill 0.4) (layers "F.Cu" "B.Cu") (free) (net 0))
 (via (at 159.1 89) (size 0.8) (drill 0.4) (layers "F.Cu" "B.Cu") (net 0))
 (via (at 184.9 106.4) (size 0.8) (drill 0.4) (layers "F.Cu" "B.Cu") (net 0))
 (via (at 154.02 90.88) (size 0.8) (drill 0.4) (layers "F.Cu" "B.Cu") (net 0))
 (via (at 123.4 117.7) (size 0.8) (drill 0.4) (layers "F.Cu" "B.Cu") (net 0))
 (via (at 105.8 88.3) (size 0.8) (drill 0.4) (layers "F.Cu" "B.Cu") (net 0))
 (via (at 156.56 89.84) (size 0.8) (drill 0.4) (layers "F.Cu" "B.Cu") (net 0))
 (via (at 104.4 90.8) (size 0.8) (drill 0.4) (layers "F.Cu" "B.Cu") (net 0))
 (via (at 185.6 93) (size 0.8) (drill 0.4) (layers "F.Cu" "B.Cu") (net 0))
 (via (at 141.5 114.5) (size 0.8) (drill 0.4) (layers "F.Cu" "B.Cu") (free) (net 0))
 (via (at 154 108) (size 0.8) (drill 0.4) (layers "F.Cu" "B.Cu") (free) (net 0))
 (via (at 162.3 89) (size 0.8) (drill 0.4) (layers "F.Cu" "B.Cu") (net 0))
 (segment (start 179.9 94.6) (end 177.6 92.3) (width 0.25) (layer "B.Cu") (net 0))
 (segment (start 163.06 89.84) (end 163.1 89.8) (width 0.2) (layer "B.Cu") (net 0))
 (segment (start 141.32 89.48) (end 141.32 95.13) (width 0.25) (layer "B.Cu") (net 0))
 (segment (start 181.75 92.35) (end 181.75 91.41) (width 0.25) (layer "B.Cu") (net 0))
 (segment (start 144.325 117) (end 144.325 110.835) (width 0.2) (layer "B.Cu") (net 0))
 (segment (start 154.02 108.02) (end 154 108) (width 0.25) (layer "B.Cu") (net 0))
 (segment (start 159 77.2) (end 159 83.1) (width 0.25) (layer "B.Cu") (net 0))
 (segment (start 183.7 109.7) (end 183.7 106.3) (width 0.25) (layer "B.Cu") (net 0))
 (segment (start 138.78 88.68) (end 138.78 95.13) (width 0.25) (layer "B.Cu") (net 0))
 (segment (start 182.5 93.1) (end 181.75 92.35) (width 0.25) (layer "B.Cu") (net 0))
 (segment (start 159.7 78.4) (end 159.7 83.3) (width 0.25) (layer "B.Cu") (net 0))
 (segment (start 154.02 110.37) (end 154.02 108.02) (width 0.25) (layer "B.Cu") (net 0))
 (segment (start 183.7 89) (end 183.57 88.87) (width 0.25) (layer "B.Cu") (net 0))
 (segment (start 179.2 87.7) (end 179.3 87.6) (width 0.25) (layer "B.Cu") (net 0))
 (segment (start 154.02 90.88) (end 163.62 90.88) (width 0.2) (layer "B.Cu") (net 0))
 (segment (start 183.7 91.2) (end 183.7 89) (width 0.25) (layer "B.Cu") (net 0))
 (segment (start 105.155 89.545) (end 108.25 89.545) (width 0.2) (layer "B.Cu") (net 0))
 (segment (start 163.62 90.88) (end 163.9 90.6) (width 0.2) (layer "B.Cu") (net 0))
 (segment (start 153.8 89.2) (end 141.6 89.2) (width 0.25) (layer "B.Cu") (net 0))
 (segment (start 140.94 117) (end 140.94 115.06) (width 0.25) (layer "B.Cu") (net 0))
 (segment (start 138.7 88.6) (end 138.78 88.68) (width 0.25) (layer "B.Cu") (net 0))
 (segment (start 184.9 109.5) (end 184.9 106.4) (width 0.25) (layer "B.Cu") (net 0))
 (segment (start 138.4 115.83) (end 143.86 110.37) (width 0.25) (layer "B.Cu") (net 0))
 (segment (start 140.94 115.06) (end 141.5 114.5) (width 0.25) (layer "B.Cu") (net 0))
 (segment (start 179.9 117.2) (end 179.9 94.6) (width 0.25) (layer "B.Cu") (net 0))
 (segment (start 105.1 89.6) (end 105.155 89.545) (width 0.2) (layer "B.Cu") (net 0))
 (segment (start 144.325 110.835) (end 143.86 110.37) (width 0.2) (layer "B.Cu") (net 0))
 (segment (start 185.6 93) (end 182.6 93) (width 0.25) (layer "B.Cu") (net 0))
 (segment (start 159.7 83.3) (end 153.8 89.2) (width 0.25) (layer "B.Cu") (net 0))
 (segment (start 153.5 88.6) (end 138.7 88.6) (width 0.25) (layer "B.Cu") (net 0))
 (segment (start 177.6 86.6) (end 177.87 86.33) (width 0.25) (layer "B.Cu") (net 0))
 (segment (start 150.225 116.735) (end 143.86 110.37) (width 0.2) (layer "B.Cu") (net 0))
 (segment (start 182.6 93) (end 182.5 93.1) (width 0.25) (layer "B.Cu") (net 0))
 (segment (start 104.4 90.8) (end 104.415 90.815) (width 0.2) (layer "B.Cu") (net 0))
 (segment (start 124.6 117.2) (end 124.6 115.4) (width 0.2) (layer "B.Cu") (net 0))
 (segment (start 123.4 117.7) (end 123.4 114.6) (width 0.2) (layer "B.Cu") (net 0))
 (segment (start 177.6 92.3) (end 177.6 86.6) (width 0.25) (layer "B.Cu") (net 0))
 (segment (start 105.8 88.3) (end 105.825 88.275) (width 0.2) (layer "B.Cu") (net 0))
 (segment (start 159 83.1) (end 153.5 88.6) (width 0.25) (layer "B.Cu") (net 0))
 (segment (start 181.5 117.52) (end 180.22 117.52) (width 0.25) (layer "B.Cu") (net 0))
 (segment (start 179.3 87.6) (end 181.75 87.6) (width 0.25) (layer "B.Cu") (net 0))
 (segment (start 138.4 117) (end 138.4 115.83) (width 0.25) (layer "B.Cu") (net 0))
 (segment (start 103.915 92.085) (end 108.25 92.085) (width 0.2) (layer "B.Cu") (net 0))
 (segment (start 156.56 89.84) (end 163.06 89.84) (width 0.2) (layer "B.Cu") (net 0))
 (segment (start 181.7 77.2) (end 159 77.2) (width 0.25) (layer "B.Cu") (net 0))
 (segment (start 103.8 92.2) (end 103.915 92.085) (width 0.2) (layer "B.Cu") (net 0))
 (segment (start 181.7 78.47) (end 159.77 78.47) (width 0.25) (layer "B.Cu") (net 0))
 (segment (start 179.2 92.3) (end 179.2 87.7) (width 0.25) (layer "B.Cu") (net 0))
 (segment (start 182.7 109.7) (end 182.7 106.2) (width 0.25) (layer "B.Cu") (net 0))
 (segment (start 141.6 89.2) (end 141.32 89.48) (width 0.25) (layer "B.Cu") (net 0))
 (segment (start 180.22 117.52) (end 179.9 117.2) (width 0.25) (layer "B.Cu") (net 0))
 (segment (start 183.57 88.87) (end 181.75 88.87) (width 0.25) (layer "B.Cu") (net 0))
 (segment (start 104.415 90.815) (end 108.25 90.815) (width 0.2) (layer "B.Cu") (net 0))
 (segment (start 150.225 117) (end 150.225 116.735) (width 0.2) (layer "B.Cu") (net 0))
 (segment (start 177.87 86.33) (end 181.75 86.33) (width 0.25) (layer "B.Cu") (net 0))
 (segment (start 159.77 78.47) (end 159.7 78.4) (width 0.25) (layer "B.Cu") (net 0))
 (segment (start 105.825 88.275) (end 108.25 88.275) (width 0.2) (layer "B.Cu") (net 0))
 (segment (start 159.1 89) (end 162.3 89) (width 0.2) (layer "B.Cu") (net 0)))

